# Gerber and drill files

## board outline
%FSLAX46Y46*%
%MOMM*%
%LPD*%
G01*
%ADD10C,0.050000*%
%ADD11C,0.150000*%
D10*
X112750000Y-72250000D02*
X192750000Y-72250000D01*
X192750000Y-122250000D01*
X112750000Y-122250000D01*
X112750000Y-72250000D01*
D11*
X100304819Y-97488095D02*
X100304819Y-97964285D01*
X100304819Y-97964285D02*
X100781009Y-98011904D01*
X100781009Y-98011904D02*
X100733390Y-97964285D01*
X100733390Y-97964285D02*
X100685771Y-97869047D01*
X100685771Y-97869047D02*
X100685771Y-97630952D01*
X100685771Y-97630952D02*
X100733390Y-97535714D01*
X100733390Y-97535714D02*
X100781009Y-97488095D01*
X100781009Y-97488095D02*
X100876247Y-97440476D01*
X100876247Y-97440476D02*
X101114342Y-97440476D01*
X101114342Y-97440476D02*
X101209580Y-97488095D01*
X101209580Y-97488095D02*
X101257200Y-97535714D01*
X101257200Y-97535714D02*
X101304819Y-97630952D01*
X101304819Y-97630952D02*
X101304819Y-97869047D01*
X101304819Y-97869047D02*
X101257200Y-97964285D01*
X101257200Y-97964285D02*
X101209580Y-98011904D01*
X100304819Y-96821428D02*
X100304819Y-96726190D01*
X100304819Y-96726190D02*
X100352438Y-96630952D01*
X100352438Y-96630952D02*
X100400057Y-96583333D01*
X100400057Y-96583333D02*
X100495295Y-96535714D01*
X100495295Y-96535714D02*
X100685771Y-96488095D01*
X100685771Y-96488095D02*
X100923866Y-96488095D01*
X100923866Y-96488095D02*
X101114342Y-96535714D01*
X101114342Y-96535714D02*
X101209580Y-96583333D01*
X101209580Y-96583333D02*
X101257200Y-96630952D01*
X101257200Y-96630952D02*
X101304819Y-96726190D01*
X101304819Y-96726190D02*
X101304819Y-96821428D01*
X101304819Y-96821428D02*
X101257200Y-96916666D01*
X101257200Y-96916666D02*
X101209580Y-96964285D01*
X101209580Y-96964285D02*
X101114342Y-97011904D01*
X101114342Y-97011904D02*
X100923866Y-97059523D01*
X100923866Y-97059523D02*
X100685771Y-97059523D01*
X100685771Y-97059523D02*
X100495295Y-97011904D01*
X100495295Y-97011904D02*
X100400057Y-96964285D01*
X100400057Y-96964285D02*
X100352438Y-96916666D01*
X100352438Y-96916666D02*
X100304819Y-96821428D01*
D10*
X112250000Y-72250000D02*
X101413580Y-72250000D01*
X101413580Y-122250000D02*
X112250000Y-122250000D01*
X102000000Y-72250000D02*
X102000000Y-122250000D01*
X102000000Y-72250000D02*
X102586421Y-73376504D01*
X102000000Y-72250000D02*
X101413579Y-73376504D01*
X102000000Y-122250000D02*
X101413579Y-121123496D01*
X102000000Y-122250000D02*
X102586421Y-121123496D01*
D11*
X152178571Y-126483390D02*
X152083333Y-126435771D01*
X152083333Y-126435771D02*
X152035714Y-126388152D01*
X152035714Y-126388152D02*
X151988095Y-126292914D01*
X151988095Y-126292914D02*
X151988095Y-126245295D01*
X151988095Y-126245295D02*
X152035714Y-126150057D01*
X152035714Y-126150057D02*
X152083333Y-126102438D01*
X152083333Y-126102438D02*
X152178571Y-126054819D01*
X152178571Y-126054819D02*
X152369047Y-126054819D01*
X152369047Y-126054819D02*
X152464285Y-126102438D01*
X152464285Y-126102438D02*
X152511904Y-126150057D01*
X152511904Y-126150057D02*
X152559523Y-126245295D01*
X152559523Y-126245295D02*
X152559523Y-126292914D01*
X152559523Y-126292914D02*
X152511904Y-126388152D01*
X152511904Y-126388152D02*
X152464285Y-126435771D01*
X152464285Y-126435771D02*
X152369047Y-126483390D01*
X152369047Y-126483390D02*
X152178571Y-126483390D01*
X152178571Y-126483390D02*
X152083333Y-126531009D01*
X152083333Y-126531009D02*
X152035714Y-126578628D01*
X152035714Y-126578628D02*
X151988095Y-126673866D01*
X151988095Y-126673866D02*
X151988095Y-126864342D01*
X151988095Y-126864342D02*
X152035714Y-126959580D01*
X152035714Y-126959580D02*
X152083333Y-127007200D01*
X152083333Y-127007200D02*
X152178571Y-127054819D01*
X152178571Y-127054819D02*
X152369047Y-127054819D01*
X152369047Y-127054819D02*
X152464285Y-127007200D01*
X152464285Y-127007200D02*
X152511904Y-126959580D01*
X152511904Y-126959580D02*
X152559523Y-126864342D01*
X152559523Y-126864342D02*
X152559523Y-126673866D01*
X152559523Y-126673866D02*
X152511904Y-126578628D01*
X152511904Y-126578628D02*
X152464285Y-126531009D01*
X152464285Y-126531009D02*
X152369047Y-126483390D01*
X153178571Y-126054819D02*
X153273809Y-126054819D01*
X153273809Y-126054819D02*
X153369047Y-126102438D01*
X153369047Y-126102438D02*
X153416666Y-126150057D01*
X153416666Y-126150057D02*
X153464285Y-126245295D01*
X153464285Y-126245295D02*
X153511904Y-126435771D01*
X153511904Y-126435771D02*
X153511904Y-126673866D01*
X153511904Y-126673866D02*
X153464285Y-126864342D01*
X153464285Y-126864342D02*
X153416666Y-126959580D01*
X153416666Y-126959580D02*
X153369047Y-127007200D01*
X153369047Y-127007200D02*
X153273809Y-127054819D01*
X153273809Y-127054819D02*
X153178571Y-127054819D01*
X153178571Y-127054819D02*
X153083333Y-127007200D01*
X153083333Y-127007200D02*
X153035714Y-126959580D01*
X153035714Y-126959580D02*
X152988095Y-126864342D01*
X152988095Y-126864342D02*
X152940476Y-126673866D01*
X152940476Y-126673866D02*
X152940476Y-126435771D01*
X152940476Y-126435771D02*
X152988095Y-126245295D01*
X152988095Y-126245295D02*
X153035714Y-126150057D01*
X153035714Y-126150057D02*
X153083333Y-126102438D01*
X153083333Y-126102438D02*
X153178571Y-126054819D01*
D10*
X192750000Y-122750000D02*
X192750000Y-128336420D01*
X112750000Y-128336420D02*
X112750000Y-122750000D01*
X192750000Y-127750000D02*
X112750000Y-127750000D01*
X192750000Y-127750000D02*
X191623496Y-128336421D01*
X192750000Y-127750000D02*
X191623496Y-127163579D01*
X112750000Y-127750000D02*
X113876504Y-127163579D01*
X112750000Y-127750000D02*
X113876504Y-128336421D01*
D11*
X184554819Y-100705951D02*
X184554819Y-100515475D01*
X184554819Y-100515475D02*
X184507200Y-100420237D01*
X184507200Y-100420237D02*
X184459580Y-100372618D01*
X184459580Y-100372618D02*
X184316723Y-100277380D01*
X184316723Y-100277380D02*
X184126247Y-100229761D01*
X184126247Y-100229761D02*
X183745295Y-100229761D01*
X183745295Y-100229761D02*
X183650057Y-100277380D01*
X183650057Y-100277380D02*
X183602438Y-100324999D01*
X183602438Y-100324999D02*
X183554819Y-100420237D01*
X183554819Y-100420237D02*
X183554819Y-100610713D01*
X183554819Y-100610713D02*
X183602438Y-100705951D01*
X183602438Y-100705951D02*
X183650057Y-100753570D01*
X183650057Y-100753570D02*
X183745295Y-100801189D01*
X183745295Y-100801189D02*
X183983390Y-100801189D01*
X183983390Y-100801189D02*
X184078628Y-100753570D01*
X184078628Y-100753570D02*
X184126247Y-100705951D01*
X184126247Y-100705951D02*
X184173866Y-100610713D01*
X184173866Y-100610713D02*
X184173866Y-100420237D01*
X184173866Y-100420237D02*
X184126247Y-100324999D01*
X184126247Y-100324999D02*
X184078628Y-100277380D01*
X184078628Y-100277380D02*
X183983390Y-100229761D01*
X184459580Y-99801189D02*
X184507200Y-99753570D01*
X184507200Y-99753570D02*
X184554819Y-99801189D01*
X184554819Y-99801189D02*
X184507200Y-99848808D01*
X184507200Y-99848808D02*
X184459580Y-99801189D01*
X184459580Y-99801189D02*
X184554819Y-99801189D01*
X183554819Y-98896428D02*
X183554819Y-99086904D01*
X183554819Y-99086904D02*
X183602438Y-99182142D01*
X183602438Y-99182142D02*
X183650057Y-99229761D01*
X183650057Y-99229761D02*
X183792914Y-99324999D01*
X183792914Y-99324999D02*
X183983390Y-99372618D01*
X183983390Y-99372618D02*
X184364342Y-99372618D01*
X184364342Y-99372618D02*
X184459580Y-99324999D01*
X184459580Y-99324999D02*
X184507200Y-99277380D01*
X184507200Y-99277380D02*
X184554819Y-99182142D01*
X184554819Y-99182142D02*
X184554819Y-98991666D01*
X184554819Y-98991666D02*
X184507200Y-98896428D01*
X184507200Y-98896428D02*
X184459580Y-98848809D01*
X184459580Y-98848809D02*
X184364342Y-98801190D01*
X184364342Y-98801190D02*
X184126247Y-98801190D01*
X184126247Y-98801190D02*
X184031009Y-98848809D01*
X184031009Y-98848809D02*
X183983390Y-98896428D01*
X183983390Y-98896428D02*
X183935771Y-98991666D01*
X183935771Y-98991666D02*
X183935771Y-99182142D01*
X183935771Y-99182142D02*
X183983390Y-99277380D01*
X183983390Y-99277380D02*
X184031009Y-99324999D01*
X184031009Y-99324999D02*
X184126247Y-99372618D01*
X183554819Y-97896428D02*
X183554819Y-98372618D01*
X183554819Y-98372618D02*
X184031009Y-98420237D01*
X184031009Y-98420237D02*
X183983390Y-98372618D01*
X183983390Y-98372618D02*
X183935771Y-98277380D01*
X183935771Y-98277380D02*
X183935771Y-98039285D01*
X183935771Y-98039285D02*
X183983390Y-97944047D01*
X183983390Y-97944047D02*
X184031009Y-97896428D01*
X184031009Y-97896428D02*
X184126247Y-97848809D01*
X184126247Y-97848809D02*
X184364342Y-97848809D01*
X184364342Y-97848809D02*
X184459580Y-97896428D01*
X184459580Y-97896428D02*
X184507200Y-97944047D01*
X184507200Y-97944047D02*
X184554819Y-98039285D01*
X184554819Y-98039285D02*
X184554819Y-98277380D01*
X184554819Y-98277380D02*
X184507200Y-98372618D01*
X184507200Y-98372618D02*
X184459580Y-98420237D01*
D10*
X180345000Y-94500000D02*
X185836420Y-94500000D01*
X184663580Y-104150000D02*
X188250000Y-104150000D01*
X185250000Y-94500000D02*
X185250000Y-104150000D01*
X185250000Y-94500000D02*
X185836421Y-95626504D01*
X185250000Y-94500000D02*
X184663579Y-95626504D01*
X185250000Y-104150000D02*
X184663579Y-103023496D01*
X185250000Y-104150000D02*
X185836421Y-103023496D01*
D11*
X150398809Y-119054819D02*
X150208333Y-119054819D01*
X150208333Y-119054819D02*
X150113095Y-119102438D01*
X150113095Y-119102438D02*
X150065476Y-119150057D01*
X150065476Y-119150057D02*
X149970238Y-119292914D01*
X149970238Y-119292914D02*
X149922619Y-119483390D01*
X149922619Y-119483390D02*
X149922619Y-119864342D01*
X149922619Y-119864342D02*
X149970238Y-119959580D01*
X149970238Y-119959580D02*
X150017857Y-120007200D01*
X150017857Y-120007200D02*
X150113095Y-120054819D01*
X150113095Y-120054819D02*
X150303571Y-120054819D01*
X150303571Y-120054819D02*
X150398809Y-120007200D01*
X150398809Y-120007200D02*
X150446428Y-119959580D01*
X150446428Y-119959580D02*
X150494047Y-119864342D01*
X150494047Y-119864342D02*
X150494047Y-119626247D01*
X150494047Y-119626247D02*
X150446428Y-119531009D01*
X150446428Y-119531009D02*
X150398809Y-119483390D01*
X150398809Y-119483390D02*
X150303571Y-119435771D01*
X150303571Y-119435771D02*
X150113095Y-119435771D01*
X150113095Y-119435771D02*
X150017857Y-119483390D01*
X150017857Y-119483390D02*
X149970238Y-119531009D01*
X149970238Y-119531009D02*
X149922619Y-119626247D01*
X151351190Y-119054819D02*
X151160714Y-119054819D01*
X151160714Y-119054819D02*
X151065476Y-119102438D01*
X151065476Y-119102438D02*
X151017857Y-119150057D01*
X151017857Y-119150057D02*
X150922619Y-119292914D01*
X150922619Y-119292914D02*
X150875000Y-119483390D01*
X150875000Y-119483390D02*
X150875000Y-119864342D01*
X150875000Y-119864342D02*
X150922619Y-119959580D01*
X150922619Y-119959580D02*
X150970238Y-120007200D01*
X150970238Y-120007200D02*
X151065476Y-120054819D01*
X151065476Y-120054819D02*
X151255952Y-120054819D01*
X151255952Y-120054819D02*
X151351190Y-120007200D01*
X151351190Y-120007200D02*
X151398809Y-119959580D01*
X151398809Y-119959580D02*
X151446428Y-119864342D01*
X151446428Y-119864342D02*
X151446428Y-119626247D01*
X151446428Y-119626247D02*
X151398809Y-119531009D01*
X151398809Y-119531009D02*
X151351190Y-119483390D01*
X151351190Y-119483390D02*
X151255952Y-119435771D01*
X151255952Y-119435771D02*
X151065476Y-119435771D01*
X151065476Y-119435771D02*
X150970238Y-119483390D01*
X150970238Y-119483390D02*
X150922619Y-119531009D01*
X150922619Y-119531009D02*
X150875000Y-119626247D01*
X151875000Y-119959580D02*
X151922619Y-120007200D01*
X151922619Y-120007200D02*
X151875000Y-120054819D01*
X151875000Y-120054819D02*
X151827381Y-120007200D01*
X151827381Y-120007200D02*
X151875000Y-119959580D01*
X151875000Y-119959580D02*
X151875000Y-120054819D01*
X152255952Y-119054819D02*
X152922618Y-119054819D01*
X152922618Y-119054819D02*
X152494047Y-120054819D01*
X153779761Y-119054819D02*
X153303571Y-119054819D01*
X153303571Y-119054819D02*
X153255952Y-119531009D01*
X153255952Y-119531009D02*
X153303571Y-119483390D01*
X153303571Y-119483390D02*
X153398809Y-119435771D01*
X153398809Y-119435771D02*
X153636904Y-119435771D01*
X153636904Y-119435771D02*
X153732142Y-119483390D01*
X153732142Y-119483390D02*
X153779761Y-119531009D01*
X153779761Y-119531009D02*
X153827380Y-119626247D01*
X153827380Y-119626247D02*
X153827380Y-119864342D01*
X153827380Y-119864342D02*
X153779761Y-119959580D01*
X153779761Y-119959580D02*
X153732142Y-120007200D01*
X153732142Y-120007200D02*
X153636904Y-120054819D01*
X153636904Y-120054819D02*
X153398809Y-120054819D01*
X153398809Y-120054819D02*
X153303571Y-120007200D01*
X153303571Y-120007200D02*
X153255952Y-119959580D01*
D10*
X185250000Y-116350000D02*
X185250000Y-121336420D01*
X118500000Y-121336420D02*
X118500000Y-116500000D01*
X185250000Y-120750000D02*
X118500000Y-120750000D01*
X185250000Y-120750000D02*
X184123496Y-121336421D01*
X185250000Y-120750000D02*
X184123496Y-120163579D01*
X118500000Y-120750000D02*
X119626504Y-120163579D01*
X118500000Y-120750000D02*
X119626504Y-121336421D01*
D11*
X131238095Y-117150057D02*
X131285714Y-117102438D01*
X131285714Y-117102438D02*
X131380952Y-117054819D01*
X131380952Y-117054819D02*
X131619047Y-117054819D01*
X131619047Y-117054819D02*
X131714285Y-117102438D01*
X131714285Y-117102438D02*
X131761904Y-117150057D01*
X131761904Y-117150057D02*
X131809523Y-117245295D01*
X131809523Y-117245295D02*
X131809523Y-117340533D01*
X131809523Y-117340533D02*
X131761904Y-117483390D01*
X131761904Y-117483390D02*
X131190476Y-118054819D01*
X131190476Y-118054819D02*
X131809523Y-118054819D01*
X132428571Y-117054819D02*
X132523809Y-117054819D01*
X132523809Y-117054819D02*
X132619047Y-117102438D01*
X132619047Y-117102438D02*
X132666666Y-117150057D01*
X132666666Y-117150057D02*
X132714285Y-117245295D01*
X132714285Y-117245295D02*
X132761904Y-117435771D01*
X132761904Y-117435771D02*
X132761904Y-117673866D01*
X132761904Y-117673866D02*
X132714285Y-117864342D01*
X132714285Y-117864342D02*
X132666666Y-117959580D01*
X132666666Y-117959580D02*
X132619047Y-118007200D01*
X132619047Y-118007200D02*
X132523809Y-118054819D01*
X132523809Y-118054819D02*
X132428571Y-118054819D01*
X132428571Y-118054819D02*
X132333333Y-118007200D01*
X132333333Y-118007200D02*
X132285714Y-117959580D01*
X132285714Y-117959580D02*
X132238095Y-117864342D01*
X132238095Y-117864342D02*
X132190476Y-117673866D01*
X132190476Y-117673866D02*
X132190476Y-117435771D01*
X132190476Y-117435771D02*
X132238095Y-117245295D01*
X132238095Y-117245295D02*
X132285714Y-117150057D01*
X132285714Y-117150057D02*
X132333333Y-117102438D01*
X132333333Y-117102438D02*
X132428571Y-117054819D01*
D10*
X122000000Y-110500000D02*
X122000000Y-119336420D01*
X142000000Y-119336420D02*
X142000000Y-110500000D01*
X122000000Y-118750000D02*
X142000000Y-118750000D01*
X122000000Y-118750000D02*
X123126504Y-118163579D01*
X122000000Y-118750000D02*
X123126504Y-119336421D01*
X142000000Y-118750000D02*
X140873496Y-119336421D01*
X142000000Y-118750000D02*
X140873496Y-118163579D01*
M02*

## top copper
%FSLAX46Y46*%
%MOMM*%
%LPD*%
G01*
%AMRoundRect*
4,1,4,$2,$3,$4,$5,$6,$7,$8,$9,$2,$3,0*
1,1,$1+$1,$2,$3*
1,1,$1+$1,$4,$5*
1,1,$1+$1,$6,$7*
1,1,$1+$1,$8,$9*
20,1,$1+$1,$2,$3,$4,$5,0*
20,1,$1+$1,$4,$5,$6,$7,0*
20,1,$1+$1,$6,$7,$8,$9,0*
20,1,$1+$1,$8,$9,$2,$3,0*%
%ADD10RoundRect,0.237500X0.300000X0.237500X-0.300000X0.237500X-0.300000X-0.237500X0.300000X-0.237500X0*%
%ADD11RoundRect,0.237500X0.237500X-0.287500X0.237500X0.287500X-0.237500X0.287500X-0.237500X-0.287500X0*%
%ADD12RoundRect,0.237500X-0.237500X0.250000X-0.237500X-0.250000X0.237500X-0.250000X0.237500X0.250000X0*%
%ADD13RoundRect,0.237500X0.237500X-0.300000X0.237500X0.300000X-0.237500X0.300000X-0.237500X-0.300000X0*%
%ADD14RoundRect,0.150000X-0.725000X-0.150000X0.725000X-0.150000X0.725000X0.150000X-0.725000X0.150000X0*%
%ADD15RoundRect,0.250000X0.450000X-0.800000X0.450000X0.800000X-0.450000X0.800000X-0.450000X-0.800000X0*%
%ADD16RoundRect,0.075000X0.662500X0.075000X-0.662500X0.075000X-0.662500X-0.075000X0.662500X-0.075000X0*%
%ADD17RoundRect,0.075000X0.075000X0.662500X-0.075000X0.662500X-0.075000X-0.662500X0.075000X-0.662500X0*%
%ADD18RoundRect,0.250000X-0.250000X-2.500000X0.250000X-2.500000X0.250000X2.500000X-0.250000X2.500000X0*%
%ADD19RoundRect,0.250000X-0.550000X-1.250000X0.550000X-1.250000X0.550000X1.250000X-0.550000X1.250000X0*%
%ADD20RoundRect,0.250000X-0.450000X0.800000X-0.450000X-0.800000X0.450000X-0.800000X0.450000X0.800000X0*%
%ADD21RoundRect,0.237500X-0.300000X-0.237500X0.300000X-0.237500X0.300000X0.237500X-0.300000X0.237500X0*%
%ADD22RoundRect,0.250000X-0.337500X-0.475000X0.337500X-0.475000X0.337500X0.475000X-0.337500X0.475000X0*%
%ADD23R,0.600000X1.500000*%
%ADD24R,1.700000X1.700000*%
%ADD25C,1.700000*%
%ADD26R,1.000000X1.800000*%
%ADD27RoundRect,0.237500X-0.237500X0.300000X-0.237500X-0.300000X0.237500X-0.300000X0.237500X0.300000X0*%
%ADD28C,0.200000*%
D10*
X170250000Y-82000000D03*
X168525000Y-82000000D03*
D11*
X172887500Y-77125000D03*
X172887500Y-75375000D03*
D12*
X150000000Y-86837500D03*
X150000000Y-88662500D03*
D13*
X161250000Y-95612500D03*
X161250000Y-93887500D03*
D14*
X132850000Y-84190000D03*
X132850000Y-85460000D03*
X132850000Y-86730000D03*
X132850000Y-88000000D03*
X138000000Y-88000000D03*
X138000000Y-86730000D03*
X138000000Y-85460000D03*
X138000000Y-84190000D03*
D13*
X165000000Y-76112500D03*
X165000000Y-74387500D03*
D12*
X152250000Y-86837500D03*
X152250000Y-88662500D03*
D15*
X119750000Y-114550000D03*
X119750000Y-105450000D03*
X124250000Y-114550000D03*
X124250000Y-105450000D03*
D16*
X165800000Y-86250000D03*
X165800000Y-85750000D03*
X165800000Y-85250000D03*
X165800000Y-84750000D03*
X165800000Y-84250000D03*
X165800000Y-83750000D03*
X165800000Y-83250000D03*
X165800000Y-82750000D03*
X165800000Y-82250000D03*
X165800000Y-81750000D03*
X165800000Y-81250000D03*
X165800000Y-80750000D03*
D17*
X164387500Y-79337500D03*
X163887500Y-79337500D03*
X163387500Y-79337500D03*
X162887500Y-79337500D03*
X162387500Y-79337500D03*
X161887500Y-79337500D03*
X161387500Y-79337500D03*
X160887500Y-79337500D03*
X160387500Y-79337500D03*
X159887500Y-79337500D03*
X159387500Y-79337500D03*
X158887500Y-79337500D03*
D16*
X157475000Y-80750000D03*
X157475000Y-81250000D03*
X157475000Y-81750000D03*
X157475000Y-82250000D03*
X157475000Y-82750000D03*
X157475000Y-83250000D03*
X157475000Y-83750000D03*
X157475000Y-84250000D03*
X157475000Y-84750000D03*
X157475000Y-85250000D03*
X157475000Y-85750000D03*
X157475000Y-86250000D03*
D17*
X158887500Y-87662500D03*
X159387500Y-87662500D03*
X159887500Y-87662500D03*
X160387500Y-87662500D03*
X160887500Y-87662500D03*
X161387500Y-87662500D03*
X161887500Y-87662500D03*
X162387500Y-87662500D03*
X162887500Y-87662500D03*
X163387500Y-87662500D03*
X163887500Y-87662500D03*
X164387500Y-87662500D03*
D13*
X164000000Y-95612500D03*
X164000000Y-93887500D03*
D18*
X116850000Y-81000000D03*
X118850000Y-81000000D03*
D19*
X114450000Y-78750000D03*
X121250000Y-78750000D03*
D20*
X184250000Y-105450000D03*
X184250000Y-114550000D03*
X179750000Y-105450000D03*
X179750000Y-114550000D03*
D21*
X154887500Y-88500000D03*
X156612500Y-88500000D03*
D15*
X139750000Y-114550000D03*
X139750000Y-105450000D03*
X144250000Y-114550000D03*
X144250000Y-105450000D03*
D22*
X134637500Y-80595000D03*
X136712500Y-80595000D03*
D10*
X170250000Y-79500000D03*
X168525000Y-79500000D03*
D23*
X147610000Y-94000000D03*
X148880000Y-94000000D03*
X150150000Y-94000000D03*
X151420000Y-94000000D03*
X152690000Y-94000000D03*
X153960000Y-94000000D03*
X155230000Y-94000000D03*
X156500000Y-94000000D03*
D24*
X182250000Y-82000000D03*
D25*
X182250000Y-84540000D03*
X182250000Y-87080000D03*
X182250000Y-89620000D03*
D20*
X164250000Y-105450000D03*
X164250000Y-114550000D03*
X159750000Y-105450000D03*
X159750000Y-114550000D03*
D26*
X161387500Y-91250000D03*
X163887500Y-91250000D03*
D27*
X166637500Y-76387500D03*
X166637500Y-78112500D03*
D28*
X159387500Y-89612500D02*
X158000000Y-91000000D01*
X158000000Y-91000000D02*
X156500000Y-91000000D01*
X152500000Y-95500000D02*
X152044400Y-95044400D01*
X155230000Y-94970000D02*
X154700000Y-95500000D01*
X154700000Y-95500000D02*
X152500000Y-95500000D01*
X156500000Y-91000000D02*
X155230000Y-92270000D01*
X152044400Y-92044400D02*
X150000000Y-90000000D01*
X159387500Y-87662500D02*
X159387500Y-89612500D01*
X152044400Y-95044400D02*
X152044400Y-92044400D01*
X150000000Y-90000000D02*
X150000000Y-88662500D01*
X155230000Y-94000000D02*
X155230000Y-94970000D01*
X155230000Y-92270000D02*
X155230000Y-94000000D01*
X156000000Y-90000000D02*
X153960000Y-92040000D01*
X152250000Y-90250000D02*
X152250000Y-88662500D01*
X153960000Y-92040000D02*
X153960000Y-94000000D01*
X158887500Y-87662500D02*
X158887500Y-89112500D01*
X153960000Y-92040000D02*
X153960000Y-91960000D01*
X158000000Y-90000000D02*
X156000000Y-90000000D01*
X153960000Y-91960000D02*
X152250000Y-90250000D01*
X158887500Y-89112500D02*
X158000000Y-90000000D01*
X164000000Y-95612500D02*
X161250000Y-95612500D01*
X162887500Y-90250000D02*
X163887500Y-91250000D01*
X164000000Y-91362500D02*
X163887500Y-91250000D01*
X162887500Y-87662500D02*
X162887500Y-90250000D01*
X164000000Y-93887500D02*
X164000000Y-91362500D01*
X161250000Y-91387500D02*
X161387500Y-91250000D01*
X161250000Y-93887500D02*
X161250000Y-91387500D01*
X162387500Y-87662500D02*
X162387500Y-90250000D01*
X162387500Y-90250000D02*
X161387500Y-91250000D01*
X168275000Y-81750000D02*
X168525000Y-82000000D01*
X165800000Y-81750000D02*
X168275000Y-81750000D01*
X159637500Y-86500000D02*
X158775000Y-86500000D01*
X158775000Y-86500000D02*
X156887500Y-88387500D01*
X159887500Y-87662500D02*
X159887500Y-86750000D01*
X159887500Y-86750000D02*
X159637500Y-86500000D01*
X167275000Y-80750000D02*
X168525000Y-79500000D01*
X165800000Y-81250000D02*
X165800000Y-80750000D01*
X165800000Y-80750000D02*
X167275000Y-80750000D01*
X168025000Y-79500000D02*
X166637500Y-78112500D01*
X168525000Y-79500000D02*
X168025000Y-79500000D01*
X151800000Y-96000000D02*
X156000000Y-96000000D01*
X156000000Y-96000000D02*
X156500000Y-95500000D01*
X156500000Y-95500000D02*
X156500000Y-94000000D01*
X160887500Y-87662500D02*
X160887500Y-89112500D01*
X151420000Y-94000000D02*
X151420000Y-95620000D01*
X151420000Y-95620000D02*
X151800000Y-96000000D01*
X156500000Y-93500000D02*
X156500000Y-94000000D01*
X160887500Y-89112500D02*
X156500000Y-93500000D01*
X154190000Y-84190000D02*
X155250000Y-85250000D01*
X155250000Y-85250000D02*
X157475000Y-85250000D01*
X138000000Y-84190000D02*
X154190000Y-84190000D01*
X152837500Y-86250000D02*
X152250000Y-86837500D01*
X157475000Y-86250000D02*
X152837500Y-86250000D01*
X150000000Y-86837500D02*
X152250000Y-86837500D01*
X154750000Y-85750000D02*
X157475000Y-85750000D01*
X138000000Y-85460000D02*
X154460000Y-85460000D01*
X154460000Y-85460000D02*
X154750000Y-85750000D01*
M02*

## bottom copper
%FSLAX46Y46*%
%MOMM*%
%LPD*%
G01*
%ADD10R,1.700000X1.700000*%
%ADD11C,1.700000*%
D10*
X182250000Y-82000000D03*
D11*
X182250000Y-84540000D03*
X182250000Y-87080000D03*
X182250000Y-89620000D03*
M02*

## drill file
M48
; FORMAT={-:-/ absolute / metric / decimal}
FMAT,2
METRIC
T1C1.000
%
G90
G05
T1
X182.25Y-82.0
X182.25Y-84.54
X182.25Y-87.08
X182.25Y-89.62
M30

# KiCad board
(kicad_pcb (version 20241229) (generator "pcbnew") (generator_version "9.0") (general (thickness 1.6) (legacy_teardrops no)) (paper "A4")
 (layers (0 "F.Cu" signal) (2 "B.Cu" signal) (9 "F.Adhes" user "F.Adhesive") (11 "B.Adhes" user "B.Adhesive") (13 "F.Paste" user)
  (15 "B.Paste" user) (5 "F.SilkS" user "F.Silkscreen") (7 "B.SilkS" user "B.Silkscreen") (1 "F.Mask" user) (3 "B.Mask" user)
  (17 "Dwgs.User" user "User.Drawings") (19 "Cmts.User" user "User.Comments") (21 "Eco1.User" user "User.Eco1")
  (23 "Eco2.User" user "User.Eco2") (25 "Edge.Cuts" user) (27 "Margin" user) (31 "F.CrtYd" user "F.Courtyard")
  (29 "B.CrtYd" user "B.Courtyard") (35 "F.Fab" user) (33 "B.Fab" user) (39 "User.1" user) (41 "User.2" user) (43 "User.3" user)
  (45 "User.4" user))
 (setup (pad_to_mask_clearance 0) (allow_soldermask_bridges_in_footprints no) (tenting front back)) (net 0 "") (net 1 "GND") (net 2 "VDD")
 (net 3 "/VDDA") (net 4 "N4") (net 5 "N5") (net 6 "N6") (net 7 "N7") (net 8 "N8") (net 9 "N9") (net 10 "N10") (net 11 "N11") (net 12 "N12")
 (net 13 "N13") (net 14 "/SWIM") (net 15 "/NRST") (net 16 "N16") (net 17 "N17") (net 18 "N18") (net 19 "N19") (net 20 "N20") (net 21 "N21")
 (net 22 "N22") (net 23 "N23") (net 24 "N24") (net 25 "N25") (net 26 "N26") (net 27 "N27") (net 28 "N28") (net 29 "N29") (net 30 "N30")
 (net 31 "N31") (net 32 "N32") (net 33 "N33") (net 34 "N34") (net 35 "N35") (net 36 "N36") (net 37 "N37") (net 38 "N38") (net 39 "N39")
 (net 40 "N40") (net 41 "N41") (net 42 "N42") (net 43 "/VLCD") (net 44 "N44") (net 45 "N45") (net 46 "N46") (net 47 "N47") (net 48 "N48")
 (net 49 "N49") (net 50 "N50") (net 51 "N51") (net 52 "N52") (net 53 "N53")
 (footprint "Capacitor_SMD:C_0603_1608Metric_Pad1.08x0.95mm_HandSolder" (layer "F.Cu") (at 169.3875 82 180)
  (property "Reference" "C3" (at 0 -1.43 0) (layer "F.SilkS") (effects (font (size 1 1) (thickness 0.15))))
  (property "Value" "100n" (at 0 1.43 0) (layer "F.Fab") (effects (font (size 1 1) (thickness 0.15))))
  (pad "1" smd roundrect (at -0.8625 0 180) (size 1.075 0.95) (layers "F.Cu" "F.Mask" "F.Paste") (roundrect_rratio 0.25) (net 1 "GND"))
  (pad "2" smd roundrect (at 0.8625 0 180) (size 1.075 0.95) (layers "F.Cu" "F.Mask" "F.Paste") (roundrect_rratio 0.25) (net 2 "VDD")))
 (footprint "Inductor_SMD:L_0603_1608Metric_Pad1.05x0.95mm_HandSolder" (layer "F.Cu") (at 172.8875 76.25 90)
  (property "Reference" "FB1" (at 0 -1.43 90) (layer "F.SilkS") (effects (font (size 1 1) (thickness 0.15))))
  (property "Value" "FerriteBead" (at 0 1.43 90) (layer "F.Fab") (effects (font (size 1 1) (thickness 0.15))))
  (pad "1" smd roundrect (at -0.875 0 90) (size 1.05 0.95) (layers "F.Cu" "F.Mask" "F.Paste") (roundrect_rratio 0.25) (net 2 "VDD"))
  (pad "2" smd roundrect (at 0.875 0 90) (size 1.05 0.95) (layers "F.Cu" "F.Mask" "F.Paste") (roundrect_rratio 0.25) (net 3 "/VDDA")))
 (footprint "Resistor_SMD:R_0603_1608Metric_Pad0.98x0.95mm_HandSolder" (layer "F.Cu") (at 150 87.75 -90)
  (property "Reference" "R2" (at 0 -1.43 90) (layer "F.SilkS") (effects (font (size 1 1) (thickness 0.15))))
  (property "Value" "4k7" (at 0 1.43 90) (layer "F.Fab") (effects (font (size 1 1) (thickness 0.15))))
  (pad "1" smd roundrect (at -0.9125 0 270) (size 0.975 0.95) (layers "F.Cu" "F.Mask" "F.Paste") (roundrect_rratio 0.25) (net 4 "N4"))
  (pad "2" smd roundrect (at 0.9125 0 270) (size 0.975 0.95) (layers "F.Cu" "F.Mask" "F.Paste") (roundrect_rratio 0.25) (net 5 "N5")))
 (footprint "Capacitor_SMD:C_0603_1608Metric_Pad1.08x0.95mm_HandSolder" (layer "F.Cu") (at 161.25 94.75 90)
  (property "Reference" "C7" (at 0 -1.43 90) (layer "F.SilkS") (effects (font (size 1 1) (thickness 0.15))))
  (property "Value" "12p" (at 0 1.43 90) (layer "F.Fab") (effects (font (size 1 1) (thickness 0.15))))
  (pad "1" smd roundrect (at -0.8625 0 90) (size 1.075 0.95) (layers "F.Cu" "F.Mask" "F.Paste") (roundrect_rratio 0.25) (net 1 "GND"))
  (pad "2" smd roundrect (at 0.8625 0 90) (size 1.075 0.95) (layers "F.Cu" "F.Mask" "F.Paste") (roundrect_rratio 0.25) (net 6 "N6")))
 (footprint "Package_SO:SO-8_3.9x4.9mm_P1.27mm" (layer "F.Cu") (at 135.425 86.095)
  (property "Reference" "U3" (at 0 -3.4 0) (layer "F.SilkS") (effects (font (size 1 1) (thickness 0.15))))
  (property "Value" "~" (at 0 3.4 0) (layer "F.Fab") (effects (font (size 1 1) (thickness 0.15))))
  (pad "1" smd roundrect (at -2.575 -1.905) (size 1.75 0.6) (layers "F.Cu" "F.Mask" "F.Paste") (roundrect_rratio 0.25) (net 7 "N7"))
  (pad "2" smd roundrect (at -2.575 -0.635) (size 1.75 0.6) (layers "F.Cu" "F.Mask" "F.Paste") (roundrect_rratio 0.25) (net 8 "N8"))
  (pad "3" smd roundrect (at -2.575 0.635) (size 1.75 0.6) (layers "F.Cu" "F.Mask" "F.Paste") (roundrect_rratio 0.25) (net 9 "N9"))
  (pad "4" smd roundrect (at -2.575 1.905) (size 1.75 0.6) (layers "F.Cu" "F.Mask" "F.Paste") (roundrect_rratio 0.25) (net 1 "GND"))
  (pad "5" smd roundrect (at 2.575 1.905) (size 1.75 0.6) (layers "F.Cu" "F.Mask" "F.Paste") (roundrect_rratio 0.25) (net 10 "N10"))
  (pad "6" smd roundrect (at 2.575 0.635) (size 1.75 0.6) (layers "F.Cu" "F.Mask" "F.Paste") (roundrect_rratio 0.25) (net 5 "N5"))
  (pad "7" smd roundrect (at 2.575 -0.635) (size 1.75 0.6) (layers "F.Cu" "F.Mask" "F.Paste") (roundrect_rratio 0.25) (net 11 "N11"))
  (pad "8" smd roundrect (at 2.575 -1.905) (size 1.75 0.6) (layers "F.Cu" "F.Mask" "F.Paste") (roundrect_rratio 0.25) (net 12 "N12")))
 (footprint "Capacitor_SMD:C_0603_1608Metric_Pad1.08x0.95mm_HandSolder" (layer "F.Cu") (at 165 75.25 90)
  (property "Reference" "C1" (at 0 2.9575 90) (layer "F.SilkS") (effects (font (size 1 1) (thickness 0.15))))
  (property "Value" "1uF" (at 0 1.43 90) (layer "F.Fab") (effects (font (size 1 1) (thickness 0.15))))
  (pad "1" smd roundrect (at -0.8625 0 90) (size 1.075 0.95) (layers "F.Cu" "F.Mask" "F.Paste") (roundrect_rratio 0.25) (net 1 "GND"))
  (pad "2" smd roundrect (at 0.8625 0 90) (size 1.075 0.95) (layers "F.Cu" "F.Mask" "F.Paste") (roundrect_rratio 0.25) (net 2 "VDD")))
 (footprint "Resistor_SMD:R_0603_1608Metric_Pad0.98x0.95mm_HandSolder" (layer "F.Cu") (at 152.25 87.75 -90)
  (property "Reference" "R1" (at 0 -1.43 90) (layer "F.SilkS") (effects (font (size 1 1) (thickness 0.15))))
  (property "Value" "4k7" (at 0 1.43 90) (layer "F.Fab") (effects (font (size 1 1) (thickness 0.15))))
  (pad "1" smd roundrect (at -0.9125 0 270) (size 0.975 0.95) (layers "F.Cu" "F.Mask" "F.Paste") (roundrect_rratio 0.25) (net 4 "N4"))
  (pad "2" smd roundrect (at 0.9125 0 270) (size 0.975 0.95) (layers "F.Cu" "F.Mask" "F.Paste") (roundrect_rratio 0.25) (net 10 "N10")))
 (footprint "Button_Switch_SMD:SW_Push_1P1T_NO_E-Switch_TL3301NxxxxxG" (layer "F.Cu") (at 122 110 90)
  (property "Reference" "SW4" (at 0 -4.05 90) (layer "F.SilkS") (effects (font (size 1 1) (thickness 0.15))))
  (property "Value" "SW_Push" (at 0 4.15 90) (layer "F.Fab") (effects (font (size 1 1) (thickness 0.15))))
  (pad "1" smd roundrect (at -4.55 -2.25 90) (size 2.1 1.4) (layers "F.Cu" "F.Mask" "F.Paste") (roundrect_rratio 0.1785714286) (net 1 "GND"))
  (pad "1" smd roundrect (at 4.55 -2.25 90) (size 2.1 1.4) (layers "F.Cu" "F.Mask" "F.Paste") (roundrect_rratio 0.1785714286) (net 1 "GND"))
  (pad "2" smd roundrect (at -4.55 2.25 90) (size 2.1 1.4) (layers "F.Cu" "F.Mask" "F.Paste") (roundrect_rratio 0.1785714286) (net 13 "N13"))
  (pad "2" smd roundrect (at 4.55 2.25 90) (size 2.1 1.4) (layers "F.Cu" "F.Mask" "F.Paste") (roundrect_rratio 0.1785714286) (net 13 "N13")))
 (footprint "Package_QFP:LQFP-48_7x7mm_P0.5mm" (layer "F.Cu") (at 161.6375 83.5 180)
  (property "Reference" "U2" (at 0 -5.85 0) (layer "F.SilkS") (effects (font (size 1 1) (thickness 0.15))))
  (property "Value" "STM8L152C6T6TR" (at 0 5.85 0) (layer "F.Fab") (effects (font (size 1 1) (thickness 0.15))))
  (pad "1" smd roundrect (at -4.1625 -2.75 180) (size 1.475 0.3) (layers "F.Cu" "F.Mask" "F.Paste") (roundrect_rratio 0.25) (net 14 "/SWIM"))
  (pad "2" smd roundrect (at -4.1625 -2.25 180) (size 1.475 0.3) (layers "F.Cu" "F.Mask" "F.Paste") (roundrect_rratio 0.25) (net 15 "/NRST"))
  (pad "3" smd roundrect (at -4.1625 -1.75 180) (size 1.475 0.3) (layers "F.Cu" "F.Mask" "F.Paste") (roundrect_rratio 0.25) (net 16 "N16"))
  (pad "4" smd roundrect (at -4.1625 -1.25 180) (size 1.475 0.3) (layers "F.Cu" "F.Mask" "F.Paste") (roundrect_rratio 0.25) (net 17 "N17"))
  (pad "5" smd roundrect (at -4.1625 -0.75 180) (size 1.475 0.3) (layers "F.Cu" "F.Mask" "F.Paste") (roundrect_rratio 0.25) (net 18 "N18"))
  (pad "6" smd roundrect (at -4.1625 -0.25 180) (size 1.475 0.3) (layers "F.Cu" "F.Mask" "F.Paste") (roundrect_rratio 0.25) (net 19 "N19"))
  (pad "7" smd roundrect (at -4.1625 0.25 180) (size 1.475 0.3) (layers "F.Cu" "F.Mask" "F.Paste") (roundrect_rratio 0.25) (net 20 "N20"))
  (pad "8" smd roundrect (at -4.1625 0.75 180) (size 1.475 0.3) (layers "F.Cu" "F.Mask" "F.Paste") (roundrect_rratio 0.25) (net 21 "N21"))
  (pad "9" smd roundrect (at -4.1625 1.25 180) (size 1.475 0.3) (layers "F.Cu" "F.Mask" "F.Paste") (roundrect_rratio 0.25) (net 1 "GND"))
  (pad "10" smd roundrect (at -4.1625 1.75 180) (size 1.475 0.3) (layers "F.Cu" "F.Mask" "F.Paste") (roundrect_rratio 0.25) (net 2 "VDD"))
  (pad "11" smd roundrect (at -4.1625 2.25 180) (size 1.475 0.3) (layers "F.Cu" "F.Mask" "F.Paste") (roundrect_rratio 0.25) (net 3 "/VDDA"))
  (pad "12" smd roundrect (at -4.1625 2.75 180) (size 1.475 0.3) (layers "F.Cu" "F.Mask" "F.Paste") (roundrect_rratio 0.25) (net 3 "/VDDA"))
  (pad "13" smd roundrect (at -2.75 4.1625 180) (size 0.3 1.475) (layers "F.Cu" "F.Mask" "F.Paste") (roundrect_rratio 0.25) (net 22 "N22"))
  (pad "14" smd roundrect (at -2.25 4.1625 180) (size 0.3 1.475) (layers "F.Cu" "F.Mask" "F.Paste") (roundrect_rratio 0.25) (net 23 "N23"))
  (pad "15" smd roundrect (at -1.75 4.1625 180) (size 0.3 1.475) (layers "F.Cu" "F.Mask" "F.Paste") (roundrect_rratio 0.25) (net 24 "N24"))
  (pad "16" smd roundrect (at -1.25 4.1625 180) (size 0.3 1.475) (layers "F.Cu" "F.Mask" "F.Paste") (roundrect_rratio 0.25) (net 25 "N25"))
  (pad "17" smd roundrect (at -0.75 4.1625 180) (size 0.3 1.475) (layers "F.Cu" "F.Mask" "F.Paste") (roundrect_rratio 0.25) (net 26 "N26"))
  (pad "18" smd roundrect (at -0.25 4.1625 180) (size 0.3 1.475) (layers "F.Cu" "F.Mask" "F.Paste") (roundrect_rratio 0.25) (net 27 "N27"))
  (pad "19" smd roundrect (at 0.25 4.1625 180) (size 0.3 1.475) (layers "F.Cu" "F.Mask" "F.Paste") (roundrect_rratio 0.25) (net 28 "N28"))
  (pad "20" smd roundrect (at 0.75 4.1625 180) (size 0.3 1.475) (layers "F.Cu" "F.Mask" "F.Paste") (roundrect_rratio 0.25) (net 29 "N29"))
  (pad "21" smd roundrect (at 1.25 4.1625 180) (size 0.3 1.475) (layers "F.Cu" "F.Mask" "F.Paste") (roundrect_rratio 0.25) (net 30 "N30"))
  (pad "22" smd roundrect (at 1.75 4.1625 180) (size 0.3 1.475) (layers "F.Cu" "F.Mask" "F.Paste") (roundrect_rratio 0.25) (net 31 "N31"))
  (pad "23" smd roundrect (at 2.25 4.1625 180) (size 0.3 1.475) (layers "F.Cu" "F.Mask" "F.Paste") (roundrect_rratio 0.25) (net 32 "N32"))
  (pad "24" smd roundrect (at 2.75 4.1625 180) (size 0.3 1.475) (layers "F.Cu" "F.Mask" "F.Paste") (roundrect_rratio 0.25) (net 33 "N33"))
  (pad "25" smd roundrect (at 4.1625 2.75 180) (size 1.475 0.3) (layers "F.Cu" "F.Mask" "F.Paste") (roundrect_rratio 0.25) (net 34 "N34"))
  (pad "26" smd roundrect (at 4.1625 2.25 180) (size 1.475 0.3) (layers "F.Cu" "F.Mask" "F.Paste") (roundrect_rratio 0.25) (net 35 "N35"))
  (pad "27" smd roundrect (at 4.1625 1.75 180) (size 1.475 0.3) (layers "F.Cu" "F.Mask" "F.Paste") (roundrect_rratio 0.25) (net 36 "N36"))
  (pad "28" smd roundrect (at 4.1625 1.25 180) (size 1.475 0.3) (layers "F.Cu" "F.Mask" "F.Paste") (roundrect_rratio 0.25) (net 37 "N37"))
  (pad "29" smd roundrect (at 4.1625 0.75 180) (size 1.475 0.3) (layers "F.Cu" "F.Mask" "F.Paste") (roundrect_rratio 0.25) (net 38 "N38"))
  (pad "30" smd roundrect (at 4.1625 0.25 180) (size 1.475 0.3) (layers "F.Cu" "F.Mask" "F.Paste") (roundrect_rratio 0.25) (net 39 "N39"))
  (pad "31" smd roundrect (at 4.1625 -0.25 180) (size 1.475 0.3) (layers "F.Cu" "F.Mask" "F.Paste") (roundrect_rratio 0.25) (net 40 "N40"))
  (pad "32" smd roundrect (at 4.1625 -0.75 180) (size 1.475 0.3) (layers "F.Cu" "F.Mask" "F.Paste") (roundrect_rratio 0.25) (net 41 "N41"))
  (pad "33" smd roundrect (at 4.1625 -1.25 180) (size 1.475 0.3) (layers "F.Cu" "F.Mask" "F.Paste") (roundrect_rratio 0.25) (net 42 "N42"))
  (pad "34" smd roundrect (at 4.1625 -1.75 180) (size 1.475 0.3) (layers "F.Cu" "F.Mask" "F.Paste") (roundrect_rratio 0.25) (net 12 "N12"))
  (pad "35" smd roundrect (at 4.1625 -2.25 180) (size 1.475 0.3) (layers "F.Cu" "F.Mask" "F.Paste") (roundrect_rratio 0.25) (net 11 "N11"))
  (pad "36" smd roundrect (at 4.1625 -2.75 180) (size 1.475 0.3) (layers "F.Cu" "F.Mask" "F.Paste") (roundrect_rratio 0.25) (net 4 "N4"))
  (pad "37" smd roundrect (at 2.75 -4.1625 180) (size 0.3 1.475) (layers "F.Cu" "F.Mask" "F.Paste") (roundrect_rratio 0.25) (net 10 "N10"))
  (pad "38" smd roundrect (at 2.25 -4.1625 180) (size 0.3 1.475) (layers "F.Cu" "F.Mask" "F.Paste") (roundrect_rratio 0.25) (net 5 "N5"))
  (pad "39" smd roundrect (at 1.75 -4.1625 180) (size 0.3 1.475) (layers "F.Cu" "F.Mask" "F.Paste") (roundrect_rratio 0.25) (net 2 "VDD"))
  (pad "40" smd roundrect (at 1.25 -4.1625 180) (size 0.3 1.475) (layers "F.Cu" "F.Mask" "F.Paste") (roundrect_rratio 0.25) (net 1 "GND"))
  (pad "41" smd roundrect (at 0.75 -4.1625 180) (size 0.3 1.475) (layers "F.Cu" "F.Mask" "F.Paste") (roundrect_rratio 0.25) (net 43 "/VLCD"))
  (pad "42" smd roundrect (at 0.25 -4.1625 180) (size 0.3 1.475) (layers "F.Cu" "F.Mask" "F.Paste") (roundrect_rratio 0.25) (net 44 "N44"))
  (pad "43" smd roundrect (at -0.25 -4.1625 180) (size 0.3 1.475) (layers "F.Cu" "F.Mask" "F.Paste") (roundrect_rratio 0.25) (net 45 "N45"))
  (pad "44" smd roundrect (at -0.75 -4.1625 180) (size 0.3 1.475) (layers "F.Cu" "F.Mask" "F.Paste") (roundrect_rratio 0.25) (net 6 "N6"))
  (pad "45" smd roundrect (at -1.25 -4.1625 180) (size 0.3 1.475) (layers "F.Cu" "F.Mask" "F.Paste") (roundrect_rratio 0.25) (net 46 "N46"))
  (pad "46" smd roundrect (at -1.75 -4.1625 180) (size 0.3 1.475) (layers "F.Cu" "F.Mask" "F.Paste") (roundrect_rratio 0.25) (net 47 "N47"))
  (pad "47" smd roundrect (at -2.25 -4.1625 180) (size 0.3 1.475) (layers "F.Cu" "F.Mask" "F.Paste") (roundrect_rratio 0.25) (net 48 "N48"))
  (pad "48" smd roundrect (at -2.75 -4.1625 180) (size 0.3 1.475) (layers "F.Cu" "F.Mask" "F.Paste") (roundrect_rratio 0.25) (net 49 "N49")))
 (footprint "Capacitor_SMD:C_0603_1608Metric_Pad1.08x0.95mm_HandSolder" (layer "F.Cu") (at 164 94.75 90)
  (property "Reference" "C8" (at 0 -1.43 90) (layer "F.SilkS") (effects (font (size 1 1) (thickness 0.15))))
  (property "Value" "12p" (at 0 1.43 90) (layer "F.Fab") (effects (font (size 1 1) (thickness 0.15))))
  (pad "1" smd roundrect (at -0.8625 0 90) (size 1.075 0.95) (layers "F.Cu" "F.Mask" "F.Paste") (roundrect_rratio 0.25) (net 1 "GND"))
  (pad "2" smd roundrect (at 0.8625 0 90) (size 1.075 0.95) (layers "F.Cu" "F.Mask" "F.Paste") (roundrect_rratio 0.25) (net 46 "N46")))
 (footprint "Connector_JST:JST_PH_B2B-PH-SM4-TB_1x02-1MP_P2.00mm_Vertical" (layer "F.Cu") (at 117.85 80.5)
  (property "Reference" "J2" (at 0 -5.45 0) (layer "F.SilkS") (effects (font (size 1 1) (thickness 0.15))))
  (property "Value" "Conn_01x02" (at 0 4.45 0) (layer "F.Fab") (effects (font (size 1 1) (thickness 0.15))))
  (pad "1" smd roundrect (at -1 0.5) (size 1 5.5) (layers "F.Cu" "F.Mask" "F.Paste") (roundrect_rratio 0.25) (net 1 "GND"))
  (pad "2" smd roundrect (at 1 0.5) (size 1 5.5) (layers "F.Cu" "F.Mask" "F.Paste") (roundrect_rratio 0.25) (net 2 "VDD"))
  (pad "MP" smd roundrect (at -3.4 -1.75) (size 1.6 3) (layers "F.Cu" "F.Mask" "F.Paste") (roundrect_rratio 0.15625))
  (pad "MP" smd roundrect (at 3.4 -1.75) (size 1.6 3) (layers "F.Cu" "F.Mask" "F.Paste") (roundrect_rratio 0.15625)))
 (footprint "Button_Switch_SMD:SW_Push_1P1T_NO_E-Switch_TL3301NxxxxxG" (layer "F.Cu") (at 182 110 -90)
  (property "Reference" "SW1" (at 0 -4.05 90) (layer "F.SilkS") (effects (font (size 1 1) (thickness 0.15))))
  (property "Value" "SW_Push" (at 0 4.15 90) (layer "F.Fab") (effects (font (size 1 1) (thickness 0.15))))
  (pad "1" smd roundrect (at -4.55 -2.25 270) (size 2.1 1.4) (layers "F.Cu" "F.Mask" "F.Paste") (roundrect_rratio 0.1785714286)
   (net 1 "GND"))
  (pad "1" smd roundrect (at 4.55 -2.25 270) (size 2.1 1.4) (layers "F.Cu" "F.Mask" "F.Paste") (roundrect_rratio 0.1785714286) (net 1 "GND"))
  (pad "2" smd roundrect (at -4.55 2.25 270) (size 2.1 1.4) (layers "F.Cu" "F.Mask" "F.Paste") (roundrect_rratio 0.1785714286)
   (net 49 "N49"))
  (pad "2" smd roundrect (at 4.55 2.25 270) (size 2.1 1.4) (layers "F.Cu" "F.Mask" "F.Paste") (roundrect_rratio 0.1785714286) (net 49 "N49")))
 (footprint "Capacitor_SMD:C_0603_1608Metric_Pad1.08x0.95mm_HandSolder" (layer "F.Cu") (at 155.75 88.5)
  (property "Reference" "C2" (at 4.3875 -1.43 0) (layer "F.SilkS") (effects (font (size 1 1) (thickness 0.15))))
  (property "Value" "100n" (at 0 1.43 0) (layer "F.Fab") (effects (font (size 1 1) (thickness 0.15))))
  (pad "1" smd roundrect (at -0.8625 0) (size 1.075 0.95) (layers "F.Cu" "F.Mask" "F.Paste") (roundrect_rratio 0.25) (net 1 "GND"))
  (pad "2" smd roundrect (at 0.8625 0) (size 1.075 0.95) (layers "F.Cu" "F.Mask" "F.Paste") (roundrect_rratio 0.25) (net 2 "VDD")))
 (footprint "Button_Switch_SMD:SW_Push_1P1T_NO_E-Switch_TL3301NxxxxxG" (layer "F.Cu") (at 142 110 90)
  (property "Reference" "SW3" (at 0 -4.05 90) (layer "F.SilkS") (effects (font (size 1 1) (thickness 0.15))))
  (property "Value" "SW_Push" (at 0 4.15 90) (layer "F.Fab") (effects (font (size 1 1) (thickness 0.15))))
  (pad "1" smd roundrect (at -4.55 -2.25 90) (size 2.1 1.4) (layers "F.Cu" "F.Mask" "F.Paste") (roundrect_rratio 0.1785714286) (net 1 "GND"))
  (pad "1" smd roundrect (at 4.55 -2.25 90) (size 2.1 1.4) (layers "F.Cu" "F.Mask" "F.Paste") (roundrect_rratio 0.1785714286) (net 1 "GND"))
  (pad "2" smd roundrect (at -4.55 2.25 90) (size 2.1 1.4) (layers "F.Cu" "F.Mask" "F.Paste") (roundrect_rratio 0.1785714286) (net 48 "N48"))
  (pad "2" smd roundrect (at 4.55 2.25 90) (size 2.1 1.4) (layers "F.Cu" "F.Mask" "F.Paste") (roundrect_rratio 0.1785714286) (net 48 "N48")))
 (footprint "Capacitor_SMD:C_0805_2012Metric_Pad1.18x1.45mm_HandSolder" (layer "F.Cu") (at 135.675 80.595)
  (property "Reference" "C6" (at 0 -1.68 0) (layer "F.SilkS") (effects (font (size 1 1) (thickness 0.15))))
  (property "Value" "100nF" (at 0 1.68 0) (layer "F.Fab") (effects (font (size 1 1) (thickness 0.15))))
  (pad "1" smd roundrect (at -1.0375 0) (size 1.175 1.45) (layers "F.Cu" "F.Mask" "F.Paste") (roundrect_rratio 0.212766) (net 1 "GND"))
  (pad "2" smd roundrect (at 1.0375 0) (size 1.175 1.45) (layers "F.Cu" "F.Mask" "F.Paste") (roundrect_rratio 0.212766) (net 12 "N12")))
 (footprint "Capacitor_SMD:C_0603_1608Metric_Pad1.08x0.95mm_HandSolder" (layer "F.Cu") (at 169.3875 79.5 180)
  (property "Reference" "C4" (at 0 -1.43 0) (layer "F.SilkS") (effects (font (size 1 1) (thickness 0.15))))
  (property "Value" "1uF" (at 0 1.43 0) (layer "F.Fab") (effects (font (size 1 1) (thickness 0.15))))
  (pad "1" smd roundrect (at -0.8625 0 180) (size 1.075 0.95) (layers "F.Cu" "F.Mask" "F.Paste") (roundrect_rratio 0.25) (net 1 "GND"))
  (pad "2" smd roundrect (at 0.8625 0 180) (size 1.075 0.95) (layers "F.Cu" "F.Mask" "F.Paste") (roundrect_rratio 0.25) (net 3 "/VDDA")))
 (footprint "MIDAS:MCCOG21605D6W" (layer "F.Cu") (at 152.055 83.6)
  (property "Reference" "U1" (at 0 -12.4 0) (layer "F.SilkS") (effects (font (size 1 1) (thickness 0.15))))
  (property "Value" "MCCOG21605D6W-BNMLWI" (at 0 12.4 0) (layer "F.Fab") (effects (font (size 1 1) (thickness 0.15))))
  (pad "1" smd rect (at -4.445 10.4) (size 0.6 1.5) (layers "F.Cu" "F.Mask" "F.Paste") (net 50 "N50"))
  (pad "2" smd rect (at -3.175 10.4) (size 0.6 1.5) (layers "F.Cu" "F.Mask" "F.Paste") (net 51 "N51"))
  (pad "3" smd rect (at -1.905 10.4) (size 0.6 1.5) (layers "F.Cu" "F.Mask" "F.Paste") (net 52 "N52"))
  (pad "4" smd rect (at -0.635 10.4) (size 0.6 1.5) (layers "F.Cu" "F.Mask" "F.Paste") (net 43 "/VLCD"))
  (pad "5" smd rect (at 0.635 10.4) (size 0.6 1.5) (layers "F.Cu" "F.Mask" "F.Paste") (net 1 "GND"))
  (pad "6" smd rect (at 1.905 10.4) (size 0.6 1.5) (layers "F.Cu" "F.Mask" "F.Paste") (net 10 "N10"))
  (pad "7" smd rect (at 3.175 10.4) (size 0.6 1.5) (layers "F.Cu" "F.Mask" "F.Paste") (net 5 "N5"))
  (pad "8" smd rect (at 4.445 10.4) (size 0.6 1.5) (layers "F.Cu" "F.Mask" "F.Paste") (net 43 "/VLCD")))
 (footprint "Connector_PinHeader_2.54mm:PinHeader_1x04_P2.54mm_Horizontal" (layer "F.Cu") (at 182.25 82)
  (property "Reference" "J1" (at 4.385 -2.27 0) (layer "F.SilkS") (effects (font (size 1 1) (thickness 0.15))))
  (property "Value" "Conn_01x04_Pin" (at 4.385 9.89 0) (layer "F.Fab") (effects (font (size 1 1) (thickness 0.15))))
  (pad "1" thru_hole rect (at 0 0) (size 1.7 1.7) (drill 1) (layers "*.Cu" "*.Mask") (remove_unused_layers no) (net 15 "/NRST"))
  (pad "2" thru_hole circle (at 0 2.54) (size 1.7 1.7) (drill 1) (layers "*.Cu" "*.Mask") (remove_unused_layers no) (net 1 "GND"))
  (pad "3" thru_hole circle (at 0 5.08) (size 1.7 1.7) (drill 1) (layers "*.Cu" "*.Mask") (remove_unused_layers no) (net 14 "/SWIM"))
  (pad "4" thru_hole circle (at 0 7.62) (size 1.7 1.7) (drill 1) (layers "*.Cu" "*.Mask") (remove_unused_layers no) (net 2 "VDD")))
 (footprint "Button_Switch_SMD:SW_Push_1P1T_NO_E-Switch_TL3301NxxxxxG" (layer "F.Cu") (at 162 110 -90)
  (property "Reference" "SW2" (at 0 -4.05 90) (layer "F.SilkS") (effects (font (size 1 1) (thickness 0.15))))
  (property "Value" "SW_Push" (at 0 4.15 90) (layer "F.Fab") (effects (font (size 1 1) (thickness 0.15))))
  (pad "1" smd roundrect (at -4.55 -2.25 270) (size 2.1 1.4) (layers "F.Cu" "F.Mask" "F.Paste") (roundrect_rratio 0.1785714286)
   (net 1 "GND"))
  (pad "1" smd roundrect (at 4.55 -2.25 270) (size 2.1 1.4) (layers "F.Cu" "F.Mask" "F.Paste") (roundrect_rratio 0.1785714286) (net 1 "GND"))
  (pad "2" smd roundrect (at -4.55 2.25 270) (size 2.1 1.4) (layers "F.Cu" "F.Mask" "F.Paste") (roundrect_rratio 0.1785714286)
   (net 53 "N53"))
  (pad "2" smd roundrect (at 4.55 2.25 270) (size 2.1 1.4) (layers "F.Cu" "F.Mask" "F.Paste") (roundrect_rratio 0.1785714286) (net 53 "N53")))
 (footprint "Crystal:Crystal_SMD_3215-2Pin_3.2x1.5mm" (layer "F.Cu") (at 162.6375 91.25 180)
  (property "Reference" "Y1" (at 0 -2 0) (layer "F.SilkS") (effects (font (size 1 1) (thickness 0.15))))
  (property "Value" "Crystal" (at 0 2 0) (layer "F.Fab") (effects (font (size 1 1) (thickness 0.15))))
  (pad "1" smd rect (at 1.25 0 180) (size 1 1.8) (layers "F.Cu" "F.Mask" "F.Paste") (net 6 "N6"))
  (pad "2" smd rect (at -1.25 0 180) (size 1 1.8) (layers "F.Cu" "F.Mask" "F.Paste") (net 46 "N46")))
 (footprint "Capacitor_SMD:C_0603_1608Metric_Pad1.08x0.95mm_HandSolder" (layer "F.Cu") (at 166.6375 77.25 -90)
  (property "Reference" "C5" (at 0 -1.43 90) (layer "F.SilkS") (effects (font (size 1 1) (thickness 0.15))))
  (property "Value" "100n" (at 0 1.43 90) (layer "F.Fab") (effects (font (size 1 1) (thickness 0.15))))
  (pad "1" smd roundrect (at -0.8625 0 270) (size 1.075 0.95) (layers "F.Cu" "F.Mask" "F.Paste") (roundrect_rratio 0.25) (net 1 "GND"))
  (pad "2" smd roundrect (at 0.8625 0 270) (size 1.075 0.95) (layers "F.Cu" "F.Mask" "F.Paste") (roundrect_rratio 0.25) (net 3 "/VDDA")))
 (gr_rect (start 112.75 72.25) (end 192.75 122.25) (stroke (width 0.05) (type default)) (fill no) (layer "Edge.Cuts"))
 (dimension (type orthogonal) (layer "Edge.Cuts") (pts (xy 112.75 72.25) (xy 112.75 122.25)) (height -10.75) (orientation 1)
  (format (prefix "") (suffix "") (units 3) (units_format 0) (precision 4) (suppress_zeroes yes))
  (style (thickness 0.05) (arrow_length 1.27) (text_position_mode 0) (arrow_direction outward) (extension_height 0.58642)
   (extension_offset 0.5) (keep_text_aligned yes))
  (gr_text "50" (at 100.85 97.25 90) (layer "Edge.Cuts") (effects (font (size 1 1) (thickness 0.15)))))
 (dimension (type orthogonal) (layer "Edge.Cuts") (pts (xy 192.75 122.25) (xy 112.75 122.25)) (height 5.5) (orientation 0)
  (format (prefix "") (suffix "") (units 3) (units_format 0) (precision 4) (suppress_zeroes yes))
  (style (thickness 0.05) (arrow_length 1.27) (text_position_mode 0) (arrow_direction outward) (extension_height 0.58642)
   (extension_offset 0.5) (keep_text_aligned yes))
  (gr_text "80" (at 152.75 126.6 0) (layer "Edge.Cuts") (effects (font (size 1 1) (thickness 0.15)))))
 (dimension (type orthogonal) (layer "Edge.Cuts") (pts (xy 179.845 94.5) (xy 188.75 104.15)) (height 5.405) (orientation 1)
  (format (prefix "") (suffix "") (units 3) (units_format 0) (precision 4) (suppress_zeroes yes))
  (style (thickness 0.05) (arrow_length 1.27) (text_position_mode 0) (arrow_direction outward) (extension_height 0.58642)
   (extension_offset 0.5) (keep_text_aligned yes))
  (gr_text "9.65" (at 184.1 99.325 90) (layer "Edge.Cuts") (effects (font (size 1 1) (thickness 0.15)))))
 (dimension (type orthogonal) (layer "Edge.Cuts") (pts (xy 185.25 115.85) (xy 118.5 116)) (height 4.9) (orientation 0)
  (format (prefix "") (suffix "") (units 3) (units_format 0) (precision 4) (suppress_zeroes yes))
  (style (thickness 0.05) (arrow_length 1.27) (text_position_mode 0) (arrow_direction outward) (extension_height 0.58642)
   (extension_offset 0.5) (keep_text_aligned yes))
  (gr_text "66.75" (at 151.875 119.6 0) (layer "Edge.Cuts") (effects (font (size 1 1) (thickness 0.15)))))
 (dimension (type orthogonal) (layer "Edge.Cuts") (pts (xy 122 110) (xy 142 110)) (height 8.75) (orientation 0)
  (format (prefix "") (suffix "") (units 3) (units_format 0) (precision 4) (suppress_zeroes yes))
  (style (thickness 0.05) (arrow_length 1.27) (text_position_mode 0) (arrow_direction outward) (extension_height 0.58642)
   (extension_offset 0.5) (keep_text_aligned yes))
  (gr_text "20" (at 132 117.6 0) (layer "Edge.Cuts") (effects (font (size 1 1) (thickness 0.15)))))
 (segment (start 159.3875 89.6125) (end 158 91) (width 0.2) (layer "F.Cu") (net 5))
 (segment (start 158 91) (end 156.5 91) (width 0.2) (layer "F.Cu") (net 5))
 (segment (start 152.5 95.5) (end 152.0444 95.0444) (width 0.2) (layer "F.Cu") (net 5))
 (segment (start 155.23 94.97) (end 154.7 95.5) (width 0.2) (layer "F.Cu") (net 5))
 (segment (start 154.7 95.5) (end 152.5 95.5) (width 0.2) (layer "F.Cu") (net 5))
 (segment (start 156.5 91) (end 155.23 92.27) (width 0.2) (layer "F.Cu") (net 5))
 (segment (start 152.0444 92.0444) (end 150 90) (width 0.2) (layer "F.Cu") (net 5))
 (segment (start 159.3875 87.6625) (end 159.3875 89.6125) (width 0.2) (layer "F.Cu") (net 5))
 (segment (start 152.0444 95.0444) (end 152.0444 92.0444) (width 0.2) (layer "F.Cu") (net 5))
 (segment (start 150 90) (end 150 88.6625) (width 0.2) (layer "F.Cu") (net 5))
 (segment (start 155.23 94) (end 155.23 94.97) (width 0.2) (layer "F.Cu") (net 5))
 (segment (start 155.23 92.27) (end 155.23 94) (width 0.2) (layer "F.Cu") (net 5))
 (segment (start 156 90) (end 153.96 92.04) (width 0.2) (layer "F.Cu") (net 10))
 (segment (start 152.25 90.25) (end 152.25 88.6625) (width 0.2) (layer "F.Cu") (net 10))
 (segment (start 153.96 92.04) (end 153.96 94) (width 0.2) (layer "F.Cu") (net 10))
 (segment (start 158.8875 87.6625) (end 158.8875 89.1125) (width 0.2) (layer "F.Cu") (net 10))
 (segment (start 153.96 92.04) (end 153.96 91.96) (width 0.2) (layer "F.Cu") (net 10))
 (segment (start 158 90) (end 156 90) (width 0.2) (layer "F.Cu") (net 10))
 (segment (start 153.96 91.96) (end 152.25 90.25) (width 0.2) (layer "F.Cu") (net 10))
 (segment (start 158.8875 89.1125) (end 158 90) (width 0.2) (layer "F.Cu") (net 10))
 (segment (start 164 95.6125) (end 161.25 95.6125) (width 0.2) (layer "F.Cu") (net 1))
 (segment (start 162.8875 90.25) (end 163.8875 91.25) (width 0.2) (layer "F.Cu") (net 46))
 (segment (start 164 91.3625) (end 163.8875 91.25) (width 0.2) (layer "F.Cu") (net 46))
 (segment (start 162.8875 87.6625) (end 162.8875 90.25) (width 0.2) (layer "F.Cu") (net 46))
 (segment (start 164 93.8875) (end 164 91.3625) (width 0.2) (layer "F.Cu") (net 46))
 (segment (start 161.25 91.3875) (end 161.3875 91.25) (width 0.2) (layer "F.Cu") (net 6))
 (segment (start 161.25 93.8875) (end 161.25 91.3875) (width 0.2) (layer "F.Cu") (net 6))
 (segment (start 162.3875 87.6625) (end 162.3875 90.25) (width 0.2) (layer "F.Cu") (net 6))
 (segment (start 162.3875 90.25) (end 161.3875 91.25) (width 0.2) (layer "F.Cu") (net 6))
 (segment (start 168.275 81.75) (end 168.525 82) (width 0.2) (layer "F.Cu") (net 2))
 (segment (start 165.8 81.75) (end 168.275 81.75) (width 0.2) (layer "F.Cu") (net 2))
 (segment (start 159.6375 86.5) (end 158.775 86.5) (width 0.2) (layer "F.Cu") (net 2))
 (segment (start 158.775 86.5) (end 156.8875 88.3875) (width 0.2) (layer "F.Cu") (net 2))
 (segment (start 159.8875 87.6625) (end 159.8875 86.75) (width 0.2) (layer "F.Cu") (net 2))
 (segment (start 159.8875 86.75) (end 159.6375 86.5) (width 0.2) (layer "F.Cu") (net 2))
 (segment (start 167.275 80.75) (end 168.525 79.5) (width 0.2) (layer "F.Cu") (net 3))
 (segment (start 165.8 81.25) (end 165.8 80.75) (width 0.2) (layer "F.Cu") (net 3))
 (segment (start 165.8 80.75) (end 167.275 80.75) (width 0.2) (layer "F.Cu") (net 3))
 (segment (start 168.025 79.5) (end 166.6375 78.1125) (width 0.2) (layer "F.Cu") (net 3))
 (segment (start 168.525 79.5) (end 168.025 79.5) (width 0.2) (layer "F.Cu") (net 3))
 (segment (start 151.8 96) (end 156 96) (width 0.2) (layer "F.Cu") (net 43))
 (segment (start 156 96) (end 156.5 95.5) (width 0.2) (layer "F.Cu") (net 43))
 (segment (start 156.5 95.5) (end 156.5 94) (width 0.2) (layer "F.Cu") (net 43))
 (segment (start 160.8875 87.6625) (end 160.8875 89.1125) (width 0.2) (layer "F.Cu") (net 43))
 (segment (start 151.42 94) (end 151.42 95.62) (width 0.2) (layer "F.Cu") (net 43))
 (segment (start 151.42 95.62) (end 151.8 96) (width 0.2) (layer "F.Cu") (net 43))
 (segment (start 156.5 93.5) (end 156.5 94) (width 0.2) (layer "F.Cu") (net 43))
 (segment (start 160.8875 89.1125) (end 156.5 93.5) (width 0.2) (layer "F.Cu") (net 43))
 (segment (start 154.19 84.19) (end 155.25 85.25) (width 0.2) (layer "F.Cu") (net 12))
 (segment (start 155.25 85.25) (end 157.475 85.25) (width 0.2) (layer "F.Cu") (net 12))
 (segment (start 138 84.19) (end 154.19 84.19) (width 0.2) (layer "F.Cu") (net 12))
 (segment (start 152.8375 86.25) (end 152.25 86.8375) (width 0.2) (layer "F.Cu") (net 4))
 (segment (start 157.475 86.25) (end 152.8375 86.25) (width 0.2) (layer "F.Cu") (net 4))
 (segment (start 150 86.8375) (end 152.25 86.8375) (width 0.2) (layer "F.Cu") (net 4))
 (segment (start 154.75 85.75) (end 157.475 85.75) (width 0.2) (layer "F.Cu") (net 11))
 (segment (start 138 85.46) (end 154.46 85.46) (width 0.2) (layer "F.Cu") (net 11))
 (segment (start 154.46 85.46) (end 154.75 85.75) (width 0.2) (layer "F.Cu") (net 11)))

